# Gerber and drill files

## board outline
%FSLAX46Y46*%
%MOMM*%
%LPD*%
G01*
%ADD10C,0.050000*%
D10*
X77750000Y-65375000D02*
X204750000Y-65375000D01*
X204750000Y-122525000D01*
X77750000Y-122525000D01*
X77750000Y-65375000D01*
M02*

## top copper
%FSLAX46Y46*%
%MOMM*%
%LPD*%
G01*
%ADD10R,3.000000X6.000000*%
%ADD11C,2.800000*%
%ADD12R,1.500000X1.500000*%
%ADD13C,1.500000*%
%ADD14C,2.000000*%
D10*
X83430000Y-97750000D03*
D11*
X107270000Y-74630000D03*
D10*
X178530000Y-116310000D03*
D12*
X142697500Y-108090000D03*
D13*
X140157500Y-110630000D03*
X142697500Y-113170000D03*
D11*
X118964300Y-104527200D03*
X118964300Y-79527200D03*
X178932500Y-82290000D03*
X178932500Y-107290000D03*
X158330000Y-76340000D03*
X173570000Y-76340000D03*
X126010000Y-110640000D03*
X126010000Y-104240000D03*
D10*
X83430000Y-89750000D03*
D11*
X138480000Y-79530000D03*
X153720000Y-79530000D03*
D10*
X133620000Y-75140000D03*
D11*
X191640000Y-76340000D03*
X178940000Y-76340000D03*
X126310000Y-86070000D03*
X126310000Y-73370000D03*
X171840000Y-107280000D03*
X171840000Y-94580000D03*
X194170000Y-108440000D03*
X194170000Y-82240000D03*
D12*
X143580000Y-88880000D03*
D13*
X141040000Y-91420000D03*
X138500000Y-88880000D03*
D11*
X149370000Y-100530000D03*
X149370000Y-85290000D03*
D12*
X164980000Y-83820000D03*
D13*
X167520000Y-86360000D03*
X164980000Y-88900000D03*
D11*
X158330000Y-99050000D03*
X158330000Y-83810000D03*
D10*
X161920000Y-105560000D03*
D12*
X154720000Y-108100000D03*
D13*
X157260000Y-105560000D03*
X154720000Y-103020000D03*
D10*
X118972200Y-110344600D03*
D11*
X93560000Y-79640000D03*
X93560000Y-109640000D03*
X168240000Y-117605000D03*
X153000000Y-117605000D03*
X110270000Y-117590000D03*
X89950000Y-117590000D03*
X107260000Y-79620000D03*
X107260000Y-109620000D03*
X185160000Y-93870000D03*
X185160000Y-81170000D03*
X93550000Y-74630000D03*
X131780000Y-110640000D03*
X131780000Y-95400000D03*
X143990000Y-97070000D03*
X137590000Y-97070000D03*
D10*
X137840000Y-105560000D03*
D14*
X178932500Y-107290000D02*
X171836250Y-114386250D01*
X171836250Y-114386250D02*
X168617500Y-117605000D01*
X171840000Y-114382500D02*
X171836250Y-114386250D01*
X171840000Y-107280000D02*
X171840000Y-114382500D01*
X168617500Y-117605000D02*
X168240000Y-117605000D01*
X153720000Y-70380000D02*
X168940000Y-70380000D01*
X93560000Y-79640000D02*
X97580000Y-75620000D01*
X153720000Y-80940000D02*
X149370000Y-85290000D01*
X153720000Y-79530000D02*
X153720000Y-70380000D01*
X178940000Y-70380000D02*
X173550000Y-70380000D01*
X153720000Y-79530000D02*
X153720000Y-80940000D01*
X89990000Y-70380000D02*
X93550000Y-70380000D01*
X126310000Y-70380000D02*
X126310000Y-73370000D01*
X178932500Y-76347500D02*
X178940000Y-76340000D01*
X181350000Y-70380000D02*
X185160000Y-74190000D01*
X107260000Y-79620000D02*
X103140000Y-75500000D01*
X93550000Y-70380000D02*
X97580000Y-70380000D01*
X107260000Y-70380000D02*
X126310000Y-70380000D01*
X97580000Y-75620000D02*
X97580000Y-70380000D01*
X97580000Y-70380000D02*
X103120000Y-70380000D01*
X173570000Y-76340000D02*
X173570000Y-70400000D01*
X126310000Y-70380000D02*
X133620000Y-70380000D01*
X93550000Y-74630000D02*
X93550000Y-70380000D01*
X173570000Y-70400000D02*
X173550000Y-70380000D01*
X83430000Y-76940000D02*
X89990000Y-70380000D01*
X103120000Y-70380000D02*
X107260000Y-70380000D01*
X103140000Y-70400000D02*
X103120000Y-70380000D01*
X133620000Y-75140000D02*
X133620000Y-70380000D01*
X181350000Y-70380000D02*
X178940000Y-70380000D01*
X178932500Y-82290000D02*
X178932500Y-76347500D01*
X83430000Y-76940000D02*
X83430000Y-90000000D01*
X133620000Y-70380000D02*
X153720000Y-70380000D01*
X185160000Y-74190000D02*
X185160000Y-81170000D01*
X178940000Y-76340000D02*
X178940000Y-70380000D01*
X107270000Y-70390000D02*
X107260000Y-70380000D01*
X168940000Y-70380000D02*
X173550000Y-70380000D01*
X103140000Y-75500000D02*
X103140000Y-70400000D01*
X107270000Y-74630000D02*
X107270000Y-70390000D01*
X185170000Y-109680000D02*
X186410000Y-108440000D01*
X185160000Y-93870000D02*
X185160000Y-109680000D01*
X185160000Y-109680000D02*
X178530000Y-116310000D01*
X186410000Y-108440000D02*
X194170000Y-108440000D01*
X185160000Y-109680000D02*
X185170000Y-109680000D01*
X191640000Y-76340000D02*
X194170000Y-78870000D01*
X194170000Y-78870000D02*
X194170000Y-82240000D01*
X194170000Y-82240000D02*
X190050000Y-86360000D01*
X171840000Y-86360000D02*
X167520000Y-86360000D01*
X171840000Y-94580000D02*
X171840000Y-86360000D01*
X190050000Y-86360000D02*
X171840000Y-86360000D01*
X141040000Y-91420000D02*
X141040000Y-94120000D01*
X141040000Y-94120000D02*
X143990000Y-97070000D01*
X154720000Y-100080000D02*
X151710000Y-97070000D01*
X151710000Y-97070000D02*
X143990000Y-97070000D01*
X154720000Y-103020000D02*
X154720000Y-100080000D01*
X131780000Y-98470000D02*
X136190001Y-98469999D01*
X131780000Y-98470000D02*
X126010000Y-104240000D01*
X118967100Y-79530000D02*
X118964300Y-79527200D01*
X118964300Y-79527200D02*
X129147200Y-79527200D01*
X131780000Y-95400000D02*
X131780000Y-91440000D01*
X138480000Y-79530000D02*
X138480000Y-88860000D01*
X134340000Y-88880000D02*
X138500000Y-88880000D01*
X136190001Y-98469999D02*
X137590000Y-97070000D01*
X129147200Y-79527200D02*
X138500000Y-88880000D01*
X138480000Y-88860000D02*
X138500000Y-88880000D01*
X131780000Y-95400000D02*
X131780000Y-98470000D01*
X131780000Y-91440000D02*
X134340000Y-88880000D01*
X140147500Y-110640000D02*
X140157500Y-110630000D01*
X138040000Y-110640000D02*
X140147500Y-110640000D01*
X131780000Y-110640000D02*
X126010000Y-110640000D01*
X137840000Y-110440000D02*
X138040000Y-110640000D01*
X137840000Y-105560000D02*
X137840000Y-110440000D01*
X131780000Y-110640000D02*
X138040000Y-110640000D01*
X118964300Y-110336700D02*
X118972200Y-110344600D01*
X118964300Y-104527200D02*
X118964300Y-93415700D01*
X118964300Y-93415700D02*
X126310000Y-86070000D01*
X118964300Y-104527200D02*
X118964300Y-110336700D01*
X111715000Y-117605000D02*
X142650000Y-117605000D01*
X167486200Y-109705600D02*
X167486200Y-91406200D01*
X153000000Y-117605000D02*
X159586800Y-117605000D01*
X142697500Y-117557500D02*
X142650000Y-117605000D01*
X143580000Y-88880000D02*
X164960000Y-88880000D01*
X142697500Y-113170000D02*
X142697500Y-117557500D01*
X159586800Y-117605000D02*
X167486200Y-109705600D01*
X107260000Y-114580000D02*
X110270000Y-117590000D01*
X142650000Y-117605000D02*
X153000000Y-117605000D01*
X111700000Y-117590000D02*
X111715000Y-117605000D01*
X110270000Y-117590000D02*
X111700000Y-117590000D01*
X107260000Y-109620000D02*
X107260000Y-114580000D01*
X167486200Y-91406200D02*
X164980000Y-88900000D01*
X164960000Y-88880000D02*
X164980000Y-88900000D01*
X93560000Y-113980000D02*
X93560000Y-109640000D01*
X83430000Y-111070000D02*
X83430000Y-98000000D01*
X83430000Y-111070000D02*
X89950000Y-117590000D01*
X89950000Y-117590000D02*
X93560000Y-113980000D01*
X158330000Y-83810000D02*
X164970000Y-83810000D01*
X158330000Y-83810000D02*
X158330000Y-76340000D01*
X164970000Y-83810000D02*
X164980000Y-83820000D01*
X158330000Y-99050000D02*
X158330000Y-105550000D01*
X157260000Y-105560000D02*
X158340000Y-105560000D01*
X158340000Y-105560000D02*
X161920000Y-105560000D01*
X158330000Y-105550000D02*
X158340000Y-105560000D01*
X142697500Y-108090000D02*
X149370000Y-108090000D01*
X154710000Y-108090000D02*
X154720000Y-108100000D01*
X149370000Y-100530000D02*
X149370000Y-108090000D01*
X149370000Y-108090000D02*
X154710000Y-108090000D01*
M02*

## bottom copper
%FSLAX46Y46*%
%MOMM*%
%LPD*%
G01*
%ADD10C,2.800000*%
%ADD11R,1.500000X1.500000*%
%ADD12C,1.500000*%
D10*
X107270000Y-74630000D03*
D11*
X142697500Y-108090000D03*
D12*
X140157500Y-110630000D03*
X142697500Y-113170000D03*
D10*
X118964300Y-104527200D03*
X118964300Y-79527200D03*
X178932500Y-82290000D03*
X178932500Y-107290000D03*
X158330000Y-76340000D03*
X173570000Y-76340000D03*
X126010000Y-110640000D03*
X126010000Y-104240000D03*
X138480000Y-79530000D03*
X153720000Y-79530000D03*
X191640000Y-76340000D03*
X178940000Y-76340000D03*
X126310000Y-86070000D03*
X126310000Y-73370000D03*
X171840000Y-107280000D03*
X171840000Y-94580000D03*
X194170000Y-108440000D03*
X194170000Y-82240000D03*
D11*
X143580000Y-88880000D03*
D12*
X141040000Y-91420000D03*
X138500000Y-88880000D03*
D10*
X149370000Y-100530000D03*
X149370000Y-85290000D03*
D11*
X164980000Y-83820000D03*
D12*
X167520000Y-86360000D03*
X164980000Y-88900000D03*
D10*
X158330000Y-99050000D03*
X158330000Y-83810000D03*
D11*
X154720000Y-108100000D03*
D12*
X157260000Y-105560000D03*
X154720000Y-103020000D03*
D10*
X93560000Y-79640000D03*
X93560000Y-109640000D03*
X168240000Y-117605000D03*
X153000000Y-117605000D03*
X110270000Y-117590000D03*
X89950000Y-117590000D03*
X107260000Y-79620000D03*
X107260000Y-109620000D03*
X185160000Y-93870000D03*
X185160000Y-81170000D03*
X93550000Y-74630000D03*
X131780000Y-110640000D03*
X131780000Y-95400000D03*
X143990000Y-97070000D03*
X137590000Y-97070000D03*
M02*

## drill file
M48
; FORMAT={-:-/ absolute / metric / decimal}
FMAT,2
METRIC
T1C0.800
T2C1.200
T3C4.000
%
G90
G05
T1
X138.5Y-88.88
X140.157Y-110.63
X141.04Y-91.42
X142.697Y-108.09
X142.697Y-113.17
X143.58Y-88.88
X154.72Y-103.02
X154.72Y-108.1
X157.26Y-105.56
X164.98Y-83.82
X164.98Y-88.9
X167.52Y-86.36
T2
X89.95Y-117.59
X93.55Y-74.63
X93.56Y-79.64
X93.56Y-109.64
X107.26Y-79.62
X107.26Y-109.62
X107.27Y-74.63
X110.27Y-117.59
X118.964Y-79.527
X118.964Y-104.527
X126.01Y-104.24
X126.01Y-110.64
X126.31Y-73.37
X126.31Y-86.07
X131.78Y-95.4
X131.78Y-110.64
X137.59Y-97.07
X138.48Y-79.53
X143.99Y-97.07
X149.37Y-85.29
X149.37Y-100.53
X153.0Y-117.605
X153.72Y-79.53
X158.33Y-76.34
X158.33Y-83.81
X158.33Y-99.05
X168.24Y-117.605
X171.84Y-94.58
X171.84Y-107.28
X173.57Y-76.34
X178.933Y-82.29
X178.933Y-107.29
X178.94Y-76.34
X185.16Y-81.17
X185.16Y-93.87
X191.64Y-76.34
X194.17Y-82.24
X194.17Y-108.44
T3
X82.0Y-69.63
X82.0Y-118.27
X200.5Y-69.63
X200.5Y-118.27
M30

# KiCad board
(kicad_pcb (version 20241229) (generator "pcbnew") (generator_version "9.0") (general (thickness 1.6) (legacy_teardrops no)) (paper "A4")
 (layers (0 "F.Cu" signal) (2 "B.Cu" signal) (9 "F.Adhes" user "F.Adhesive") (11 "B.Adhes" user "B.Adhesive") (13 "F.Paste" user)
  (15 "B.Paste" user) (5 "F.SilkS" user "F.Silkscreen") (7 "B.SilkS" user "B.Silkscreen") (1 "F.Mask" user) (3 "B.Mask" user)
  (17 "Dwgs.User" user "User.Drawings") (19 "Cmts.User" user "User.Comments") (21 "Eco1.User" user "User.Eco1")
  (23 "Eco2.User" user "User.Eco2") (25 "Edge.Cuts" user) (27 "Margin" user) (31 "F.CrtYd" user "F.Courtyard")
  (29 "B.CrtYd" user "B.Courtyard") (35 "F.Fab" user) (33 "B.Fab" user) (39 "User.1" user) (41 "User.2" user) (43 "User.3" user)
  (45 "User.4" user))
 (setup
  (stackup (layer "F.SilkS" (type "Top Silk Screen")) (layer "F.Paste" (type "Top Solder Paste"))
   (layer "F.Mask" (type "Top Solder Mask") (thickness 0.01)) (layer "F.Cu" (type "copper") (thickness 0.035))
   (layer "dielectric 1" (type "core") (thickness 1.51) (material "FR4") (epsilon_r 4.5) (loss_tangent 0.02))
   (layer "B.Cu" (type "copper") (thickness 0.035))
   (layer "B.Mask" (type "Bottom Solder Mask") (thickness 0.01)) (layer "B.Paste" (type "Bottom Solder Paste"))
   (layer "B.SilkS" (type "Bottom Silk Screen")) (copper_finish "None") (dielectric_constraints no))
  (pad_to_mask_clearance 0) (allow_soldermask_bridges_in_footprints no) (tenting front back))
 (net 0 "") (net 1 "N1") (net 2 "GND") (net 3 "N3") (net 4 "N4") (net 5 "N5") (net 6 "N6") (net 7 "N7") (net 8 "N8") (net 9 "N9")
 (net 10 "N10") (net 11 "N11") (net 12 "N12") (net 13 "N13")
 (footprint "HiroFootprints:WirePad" (layer "F.Cu") (at 83.43 98)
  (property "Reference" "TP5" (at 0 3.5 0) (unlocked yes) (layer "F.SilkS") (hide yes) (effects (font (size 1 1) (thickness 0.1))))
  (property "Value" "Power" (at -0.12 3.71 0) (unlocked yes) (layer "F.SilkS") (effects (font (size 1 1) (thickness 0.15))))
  (pad "1" smd rect (at 0 -0.25) (size 3 6) (layers "F.Cu" "F.Mask" "F.Paste") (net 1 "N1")))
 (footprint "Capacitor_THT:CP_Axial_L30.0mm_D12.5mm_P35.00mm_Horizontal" (layer "F.Cu") (at 107.27 74.63 -90)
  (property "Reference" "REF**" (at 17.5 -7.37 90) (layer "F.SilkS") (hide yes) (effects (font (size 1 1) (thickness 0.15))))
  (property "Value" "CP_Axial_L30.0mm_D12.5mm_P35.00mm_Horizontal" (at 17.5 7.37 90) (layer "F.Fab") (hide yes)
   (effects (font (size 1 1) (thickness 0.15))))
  (pad "1" thru_hole circle (at 0 0 270) (size 2.8 2.8) (drill 1.2) (layers "*.Cu" "*.Mask") (remove_unused_layers no) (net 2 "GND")))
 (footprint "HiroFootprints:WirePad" (layer "F.Cu") (at 178.53 116.56)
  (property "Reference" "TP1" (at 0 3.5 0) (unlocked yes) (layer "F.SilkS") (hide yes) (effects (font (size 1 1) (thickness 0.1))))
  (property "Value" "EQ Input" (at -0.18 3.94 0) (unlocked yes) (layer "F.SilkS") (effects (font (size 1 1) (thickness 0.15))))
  (pad "1" smd rect (at 0 -0.25) (size 3 6) (layers "F.Cu" "F.Mask" "F.Paste") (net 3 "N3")))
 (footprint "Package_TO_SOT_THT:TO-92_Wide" (layer "F.Cu") (at 142.6975 108.09 -90)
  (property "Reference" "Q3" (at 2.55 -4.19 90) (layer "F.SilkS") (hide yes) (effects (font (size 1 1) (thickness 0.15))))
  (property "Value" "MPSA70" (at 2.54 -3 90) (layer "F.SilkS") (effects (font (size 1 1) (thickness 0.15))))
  (pad "1" thru_hole rect (at 0 0 270) (size 1.5 1.5) (drill 0.8) (layers "*.Cu" "*.Mask") (remove_unused_layers no) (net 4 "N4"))
  (pad "2" thru_hole circle (at 2.54 2.54 270) (size 1.5 1.5) (drill 0.8) (layers "*.Cu" "*.Mask") (remove_unused_layers no) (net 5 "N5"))
  (pad "3" thru_hole circle (at 5.08 0 270) (size 1.5 1.5) (drill 0.8) (layers "*.Cu" "*.Mask") (remove_unused_layers no) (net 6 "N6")))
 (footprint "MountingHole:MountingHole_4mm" (layer "F.Cu") (at 200.5 118.27)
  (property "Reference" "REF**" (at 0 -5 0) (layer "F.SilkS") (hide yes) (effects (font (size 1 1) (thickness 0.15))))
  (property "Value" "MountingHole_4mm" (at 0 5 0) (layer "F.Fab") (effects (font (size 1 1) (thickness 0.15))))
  (pad "" np_thru_hole circle (at 0 0) (size 4 4) (drill 4) (layers "*.Cu" "*.Mask")))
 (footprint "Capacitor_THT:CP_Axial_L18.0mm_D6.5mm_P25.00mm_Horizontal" (layer "F.Cu") (at 118.9643 104.5272 90)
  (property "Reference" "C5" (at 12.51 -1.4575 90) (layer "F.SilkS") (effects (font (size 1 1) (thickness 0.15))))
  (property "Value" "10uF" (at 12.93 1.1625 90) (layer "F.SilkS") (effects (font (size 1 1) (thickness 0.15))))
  (pad "1" thru_hole circle (at 0 0 90) (size 2.8 2.8) (drill 1.2) (layers "*.Cu" "*.Mask") (remove_unused_layers no) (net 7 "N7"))
  (pad "2" thru_hole circle (at 25 0 90) (size 2.8 2.8) (drill 1.2) (layers "*.Cu" "*.Mask") (remove_unused_layers no) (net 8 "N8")))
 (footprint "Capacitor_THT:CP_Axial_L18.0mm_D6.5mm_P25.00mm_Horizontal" (layer "F.Cu") (at 178.9325 82.29 -90)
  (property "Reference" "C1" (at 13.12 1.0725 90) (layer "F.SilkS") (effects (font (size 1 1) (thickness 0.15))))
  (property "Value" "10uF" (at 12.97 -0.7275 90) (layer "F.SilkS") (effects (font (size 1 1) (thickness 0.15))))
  (pad "1" thru_hole circle (at 0 0 270) (size 2.8 2.8) (drill 1.2) (layers "*.Cu" "*.Mask") (remove_unused_layers no) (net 2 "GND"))
  (pad "2" thru_hole circle (at 25 0 270) (size 2.8 2.8) (drill 1.2) (layers "*.Cu" "*.Mask") (remove_unused_layers no) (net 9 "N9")))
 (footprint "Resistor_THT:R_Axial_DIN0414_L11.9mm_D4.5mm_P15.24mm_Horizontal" (layer "F.Cu") (at 158.33 76.34)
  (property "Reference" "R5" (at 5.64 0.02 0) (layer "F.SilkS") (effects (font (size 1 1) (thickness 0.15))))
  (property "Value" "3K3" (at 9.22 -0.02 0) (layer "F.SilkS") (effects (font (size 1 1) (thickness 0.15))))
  (pad "1" thru_hole circle (at 0 0) (size 2.8 2.8) (drill 1.2) (layers "*.Cu" "*.Mask") (remove_unused_layers no) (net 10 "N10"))
  (pad "2" thru_hole circle (at 15.24 0) (size 2.8 2.8) (drill 1.2) (layers "*.Cu" "*.Mask") (remove_unused_layers no) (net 2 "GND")))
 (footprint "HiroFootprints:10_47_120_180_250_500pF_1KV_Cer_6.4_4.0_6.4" (layer "F.Cu") (at 126.01 110.64 90)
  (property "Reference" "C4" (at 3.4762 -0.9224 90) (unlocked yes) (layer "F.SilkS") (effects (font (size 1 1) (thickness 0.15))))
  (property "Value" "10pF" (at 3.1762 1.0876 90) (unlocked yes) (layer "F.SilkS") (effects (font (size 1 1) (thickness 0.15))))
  (pad "1" thru_hole circle (at 0 0 90) (size 2.8 2.8) (drill 1.2) (layers "*.Cu" "*.Mask") (remove_unused_layers no) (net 5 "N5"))
  (pad "2" thru_hole circle (at 6.4 0 90) (size 2.8 2.8) (drill 1.2) (layers "*.Cu" "*.Mask") (remove_unused_layers no) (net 8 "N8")))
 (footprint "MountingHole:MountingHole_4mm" (layer "F.Cu") (at 200.5 69.63)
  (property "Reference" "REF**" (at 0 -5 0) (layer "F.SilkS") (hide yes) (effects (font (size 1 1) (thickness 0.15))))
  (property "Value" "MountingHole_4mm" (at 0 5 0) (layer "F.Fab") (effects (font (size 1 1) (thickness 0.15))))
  (pad "" np_thru_hole circle (at 0 0) (size 4 4) (drill 4) (layers "*.Cu" "*.Mask")))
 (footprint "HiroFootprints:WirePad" (layer "F.Cu") (at 83.43 90)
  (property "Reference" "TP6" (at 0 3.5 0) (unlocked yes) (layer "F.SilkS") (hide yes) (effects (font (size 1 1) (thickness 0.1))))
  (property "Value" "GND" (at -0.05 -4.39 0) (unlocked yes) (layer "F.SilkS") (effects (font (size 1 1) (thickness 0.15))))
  (pad "1" smd rect (at 0 -0.25) (size 3 6) (layers "F.Cu" "F.Mask" "F.Paste") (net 2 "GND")))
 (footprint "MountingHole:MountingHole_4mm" (layer "F.Cu") (at 82 69.63)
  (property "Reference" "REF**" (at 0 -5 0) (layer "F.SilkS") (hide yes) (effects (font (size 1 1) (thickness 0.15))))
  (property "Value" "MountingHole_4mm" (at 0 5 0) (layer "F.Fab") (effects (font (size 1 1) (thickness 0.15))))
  (pad "" np_thru_hole circle (at 0 0) (size 4 4) (drill 4) (layers "*.Cu" "*.Mask")))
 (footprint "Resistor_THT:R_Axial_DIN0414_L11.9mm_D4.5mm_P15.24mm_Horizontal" (layer "F.Cu") (at 138.48 79.53)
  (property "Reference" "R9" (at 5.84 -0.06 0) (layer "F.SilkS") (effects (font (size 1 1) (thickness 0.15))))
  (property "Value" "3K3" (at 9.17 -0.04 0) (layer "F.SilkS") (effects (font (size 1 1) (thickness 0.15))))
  (pad "1" thru_hole circle (at 0 0) (size 2.8 2.8) (drill 1.2) (layers "*.Cu" "*.Mask") (remove_unused_layers no) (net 8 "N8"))
  (pad "2" thru_hole circle (at 15.24 0) (size 2.8 2.8) (drill 1.2) (layers "*.Cu" "*.Mask") (remove_unused_layers no) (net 2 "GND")))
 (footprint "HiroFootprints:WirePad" (layer "F.Cu") (at 133.62 75.39)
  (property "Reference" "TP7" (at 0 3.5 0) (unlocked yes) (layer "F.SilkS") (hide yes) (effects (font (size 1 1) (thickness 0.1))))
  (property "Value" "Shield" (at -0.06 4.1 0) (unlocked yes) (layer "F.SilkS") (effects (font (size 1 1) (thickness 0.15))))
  (pad "1" smd rect (at 0 -0.25) (size 3 6) (layers "F.Cu" "F.Mask" "F.Paste") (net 2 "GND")))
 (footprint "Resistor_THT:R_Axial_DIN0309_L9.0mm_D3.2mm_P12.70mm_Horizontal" (layer "F.Cu") (at 191.64 76.34 180)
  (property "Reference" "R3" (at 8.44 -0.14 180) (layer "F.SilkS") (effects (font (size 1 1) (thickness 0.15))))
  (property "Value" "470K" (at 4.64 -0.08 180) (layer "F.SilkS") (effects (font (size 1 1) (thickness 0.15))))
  (pad "1" thru_hole circle (at 0 0 180) (size 2.8 2.8) (drill 1.2) (layers "*.Cu" "*.Mask") (remove_unused_layers no) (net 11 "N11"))
  (pad "2" thru_hole circle (at 12.7 0 180) (size 2.8 2.8) (drill 1.2) (layers "*.Cu" "*.Mask") (remove_unused_layers no) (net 2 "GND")))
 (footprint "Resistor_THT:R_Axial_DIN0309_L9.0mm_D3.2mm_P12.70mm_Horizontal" (layer "F.Cu") (at 126.31 86.07 90)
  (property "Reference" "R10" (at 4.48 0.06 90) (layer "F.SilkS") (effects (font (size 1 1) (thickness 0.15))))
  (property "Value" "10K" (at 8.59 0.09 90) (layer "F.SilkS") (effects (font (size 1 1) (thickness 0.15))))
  (pad "1" thru_hole circle (at 0 0 90) (size 2.8 2.8) (drill 1.2) (layers "*.Cu" "*.Mask") (remove_unused_layers no) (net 7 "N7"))
  (pad "2" thru_hole circle (at 12.7 0 90) (size 2.8 2.8) (drill 1.2) (layers "*.Cu" "*.Mask") (remove_unused_layers no) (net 2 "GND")))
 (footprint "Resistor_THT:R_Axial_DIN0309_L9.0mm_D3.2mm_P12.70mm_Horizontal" (layer "F.Cu") (at 171.84 107.28 90)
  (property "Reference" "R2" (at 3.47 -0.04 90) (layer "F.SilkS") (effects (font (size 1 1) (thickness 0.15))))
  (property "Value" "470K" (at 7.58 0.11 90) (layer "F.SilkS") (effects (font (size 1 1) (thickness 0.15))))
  (pad "1" thru_hole circle (at 0 0 90) (size 2.8 2.8) (drill 1.2) (layers "*.Cu" "*.Mask") (remove_unused_layers no) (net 9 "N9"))
  (pad "2" thru_hole circle (at 12.7 0 90) (size 2.8 2.8) (drill 1.2) (layers "*.Cu" "*.Mask") (remove_unused_layers no) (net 11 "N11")))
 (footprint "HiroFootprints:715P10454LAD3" (layer "F.Cu") (at 194.17 108.44 90)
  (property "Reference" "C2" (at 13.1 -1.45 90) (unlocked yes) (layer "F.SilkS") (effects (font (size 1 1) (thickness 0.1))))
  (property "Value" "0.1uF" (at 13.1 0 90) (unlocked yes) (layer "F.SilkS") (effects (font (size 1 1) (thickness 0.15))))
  (pad "1" thru_hole circle (at 0 0 90) (size 2.8 2.8) (drill 1.2) (layers "*.Cu" "*.Mask") (remove_unused_layers no) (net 3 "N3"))
  (pad "2" thru_hole circle (at 26.2 0 90) (size 2.8 2.8) (drill 1.2) (layers "*.Cu" "*.Mask") (remove_unused_layers no) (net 11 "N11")))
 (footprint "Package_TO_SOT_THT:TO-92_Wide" (layer "F.Cu") (at 143.58 88.88 180)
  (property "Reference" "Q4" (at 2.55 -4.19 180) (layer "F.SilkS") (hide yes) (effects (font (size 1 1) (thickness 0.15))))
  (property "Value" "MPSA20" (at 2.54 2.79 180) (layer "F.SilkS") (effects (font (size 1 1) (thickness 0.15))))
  (pad "1" thru_hole rect (at 0 0 180) (size 1.5 1.5) (drill 0.8) (layers "*.Cu" "*.Mask") (remove_unused_layers no) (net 6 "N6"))
  (pad "2" thru_hole circle (at 2.54 -2.54 180) (size 1.5 1.5) (drill 0.8) (layers "*.Cu" "*.Mask") (remove_unused_layers no) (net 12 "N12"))
  (pad "3" thru_hole circle (at 5.08 0 180) (size 1.5 1.5) (drill 0.8) (layers "*.Cu" "*.Mask") (remove_unused_layers no) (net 8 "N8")))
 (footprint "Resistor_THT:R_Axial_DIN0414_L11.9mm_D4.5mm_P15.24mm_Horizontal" (layer "F.Cu") (at 149.37 100.53 90)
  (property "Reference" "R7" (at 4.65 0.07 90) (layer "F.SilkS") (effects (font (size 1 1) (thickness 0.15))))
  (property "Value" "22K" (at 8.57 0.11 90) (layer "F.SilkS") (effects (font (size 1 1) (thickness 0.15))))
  (pad "1" thru_hole circle (at 0 0 90) (size 2.8 2.8) (drill 1.2) (layers "*.Cu" "*.Mask") (remove_unused_layers no) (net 4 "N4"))
  (pad "2" thru_hole circle (at 15.24 0 90) (size 2.8 2.8) (drill 1.2) (layers "*.Cu" "*.Mask") (remove_unused_layers no) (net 2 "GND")))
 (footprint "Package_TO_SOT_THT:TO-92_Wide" (layer "F.Cu") (at 164.98 83.82 -90)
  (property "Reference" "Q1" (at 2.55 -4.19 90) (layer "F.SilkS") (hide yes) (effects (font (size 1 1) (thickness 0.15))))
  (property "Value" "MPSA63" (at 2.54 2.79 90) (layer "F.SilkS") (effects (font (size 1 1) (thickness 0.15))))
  (pad "1" thru_hole rect (at 0 0 270) (size 1.5 1.5) (drill 0.8) (layers "*.Cu" "*.Mask") (remove_unused_layers no) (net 10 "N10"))
  (pad "2" thru_hole circle (at 2.54 -2.54 270) (size 1.5 1.5) (drill 0.8) (layers "*.Cu" "*.Mask") (remove_unused_layers no) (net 11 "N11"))
  (pad "3" thru_hole circle (at 5.08 0 270) (size 1.5 1.5) (drill 0.8) (layers "*.Cu" "*.Mask") (remove_unused_layers no) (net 6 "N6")))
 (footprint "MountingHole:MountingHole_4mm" (layer "F.Cu") (at 82 118.27)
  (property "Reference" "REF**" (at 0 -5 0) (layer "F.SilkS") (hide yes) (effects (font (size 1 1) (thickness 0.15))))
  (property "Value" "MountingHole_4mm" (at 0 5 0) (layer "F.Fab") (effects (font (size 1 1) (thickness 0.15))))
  (pad "" np_thru_hole circle (at 0 0) (size 4 4) (drill 4) (layers "*.Cu" "*.Mask")))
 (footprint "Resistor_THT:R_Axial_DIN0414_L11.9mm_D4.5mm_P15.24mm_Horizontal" (layer "F.Cu") (at 158.33 99.05 90)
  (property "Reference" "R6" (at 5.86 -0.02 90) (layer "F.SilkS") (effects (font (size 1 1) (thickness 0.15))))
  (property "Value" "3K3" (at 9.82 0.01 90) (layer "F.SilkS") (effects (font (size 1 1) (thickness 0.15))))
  (pad "1" thru_hole circle (at 0 0 90) (size 2.8 2.8) (drill 1.2) (layers "*.Cu" "*.Mask") (remove_unused_layers no) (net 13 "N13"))
  (pad "2" thru_hole circle (at 15.24 0 90) (size 2.8 2.8) (drill 1.2) (layers "*.Cu" "*.Mask") (remove_unused_layers no) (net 10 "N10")))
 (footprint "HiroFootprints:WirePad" (layer "F.Cu") (at 161.92 105.81)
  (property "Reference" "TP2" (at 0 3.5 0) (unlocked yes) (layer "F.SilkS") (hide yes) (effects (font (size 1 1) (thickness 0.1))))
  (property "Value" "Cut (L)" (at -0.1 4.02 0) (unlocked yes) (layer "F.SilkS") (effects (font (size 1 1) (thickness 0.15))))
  (pad "1" smd rect (at 0 -0.25) (size 3 6) (layers "F.Cu" "F.Mask" "F.Paste") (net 13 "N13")))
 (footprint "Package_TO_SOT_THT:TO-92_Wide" (layer "F.Cu") (at 154.72 108.1 90)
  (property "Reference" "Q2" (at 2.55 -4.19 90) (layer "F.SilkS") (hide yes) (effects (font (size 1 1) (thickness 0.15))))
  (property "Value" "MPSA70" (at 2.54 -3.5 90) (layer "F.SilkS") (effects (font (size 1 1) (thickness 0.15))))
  (pad "1" thru_hole rect (at 0 0 90) (size 1.5 1.5) (drill 0.8) (layers "*.Cu" "*.Mask") (remove_unused_layers no) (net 4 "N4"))
  (pad "2" thru_hole circle (at 2.54 2.54 90) (size 1.5 1.5) (drill 0.8) (layers "*.Cu" "*.Mask") (remove_unused_layers no) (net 13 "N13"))
  (pad "3" thru_hole circle (at 5.08 0 90) (size 1.5 1.5) (drill 0.8) (layers "*.Cu" "*.Mask") (remove_unused_layers no) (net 12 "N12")))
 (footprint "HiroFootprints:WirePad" (layer "F.Cu") (at 118.9722 110.5946)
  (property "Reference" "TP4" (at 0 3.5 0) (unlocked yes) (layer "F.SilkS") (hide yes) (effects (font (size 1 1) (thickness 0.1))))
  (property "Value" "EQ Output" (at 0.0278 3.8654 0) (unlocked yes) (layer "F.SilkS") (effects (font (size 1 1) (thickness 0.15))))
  (pad "1" smd rect (at 0 -0.25) (size 3 6) (layers "F.Cu" "F.Mask" "F.Paste") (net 7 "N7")))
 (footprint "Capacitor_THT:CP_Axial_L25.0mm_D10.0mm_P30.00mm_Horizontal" (layer "F.Cu") (at 93.56 79.64 -90)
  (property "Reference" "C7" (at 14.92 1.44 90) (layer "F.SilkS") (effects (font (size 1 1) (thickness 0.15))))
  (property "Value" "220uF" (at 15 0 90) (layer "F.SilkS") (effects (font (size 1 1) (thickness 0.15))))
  (pad "1" thru_hole circle (at 0 0 270) (size 2.8 2.8) (drill 1.2) (layers "*.Cu" "*.Mask") (remove_unused_layers no) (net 2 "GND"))
  (pad "2" thru_hole circle (at 30 0 270) (size 2.8 2.8) (drill 1.2) (layers "*.Cu" "*.Mask") (remove_unused_layers no) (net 1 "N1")))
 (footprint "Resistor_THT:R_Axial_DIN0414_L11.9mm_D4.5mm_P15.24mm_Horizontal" (layer "F.Cu") (at 168.24 117.605 180)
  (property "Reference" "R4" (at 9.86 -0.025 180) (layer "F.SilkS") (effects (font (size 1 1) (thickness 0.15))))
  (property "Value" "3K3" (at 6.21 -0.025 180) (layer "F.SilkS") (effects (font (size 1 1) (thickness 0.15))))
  (pad "1" thru_hole circle (at 0 0 180) (size 2.8 2.8) (drill 1.2) (layers "*.Cu" "*.Mask") (remove_unused_layers no) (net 9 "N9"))
  (pad "2" thru_hole circle (at 15.24 0 180) (size 2.8 2.8) (drill 1.2) (layers "*.Cu" "*.Mask") (remove_unused_layers no) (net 6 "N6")))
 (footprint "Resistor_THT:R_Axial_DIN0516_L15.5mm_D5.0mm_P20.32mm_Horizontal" (layer "F.Cu") (at 110.27 117.59 180)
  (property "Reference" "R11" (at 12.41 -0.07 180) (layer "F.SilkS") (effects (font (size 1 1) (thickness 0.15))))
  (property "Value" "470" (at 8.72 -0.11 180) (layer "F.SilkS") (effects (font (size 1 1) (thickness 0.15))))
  (pad "1" thru_hole circle (at 0 0 180) (size 2.8 2.8) (drill 1.2) (layers "*.Cu" "*.Mask") (remove_unused_layers no) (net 6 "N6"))
  (pad "2" thru_hole circle (at 20.32 0 180) (size 2.8 2.8) (drill 1.2) (layers "*.Cu" "*.Mask") (remove_unused_layers no) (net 1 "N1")))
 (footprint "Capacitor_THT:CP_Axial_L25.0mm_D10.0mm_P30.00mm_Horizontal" (layer "F.Cu") (at 107.26 79.62 -90)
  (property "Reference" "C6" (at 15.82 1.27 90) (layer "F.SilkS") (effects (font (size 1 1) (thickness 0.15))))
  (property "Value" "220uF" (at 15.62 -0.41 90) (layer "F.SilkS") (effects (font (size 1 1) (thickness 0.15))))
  (pad "1" thru_hole circle (at 0 0 270) (size 2.8 2.8) (drill 1.2) (layers "*.Cu" "*.Mask") (remove_unused_layers no) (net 2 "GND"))
  (pad "2" thru_hole circle (at 30 0 270) (size 2.8 2.8) (drill 1.2) (layers "*.Cu" "*.Mask") (remove_unused_layers no) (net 6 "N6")))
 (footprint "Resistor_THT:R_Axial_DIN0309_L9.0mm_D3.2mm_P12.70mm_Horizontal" (layer "F.Cu") (at 185.16 93.87 90)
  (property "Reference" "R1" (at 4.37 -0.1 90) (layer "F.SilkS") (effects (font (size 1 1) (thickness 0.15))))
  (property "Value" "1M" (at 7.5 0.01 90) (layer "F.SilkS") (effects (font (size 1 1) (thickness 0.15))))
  (pad "1" thru_hole circle (at 0 0 90) (size 2.8 2.8) (drill 1.2) (layers "*.Cu" "*.Mask") (remove_unused_layers no) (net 3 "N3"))
  (pad "2" thru_hole circle (at 12.7 0 90) (size 2.8 2.8) (drill 1.2) (layers "*.Cu" "*.Mask") (remove_unused_layers no) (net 2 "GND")))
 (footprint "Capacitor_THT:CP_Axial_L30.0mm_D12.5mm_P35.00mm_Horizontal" (layer "F.Cu") (at 93.55 74.63 -90)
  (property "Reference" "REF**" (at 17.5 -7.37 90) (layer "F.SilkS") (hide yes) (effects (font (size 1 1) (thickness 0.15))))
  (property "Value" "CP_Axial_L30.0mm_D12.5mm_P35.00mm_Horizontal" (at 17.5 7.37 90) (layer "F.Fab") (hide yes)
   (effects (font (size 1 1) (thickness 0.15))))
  (pad "1" thru_hole circle (at 0 0 270) (size 2.8 2.8) (drill 1.2) (layers "*.Cu" "*.Mask") (remove_unused_layers no) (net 2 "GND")))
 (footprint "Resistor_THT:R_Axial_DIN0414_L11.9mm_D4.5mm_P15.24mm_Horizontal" (layer "F.Cu") (at 131.78 110.64 90)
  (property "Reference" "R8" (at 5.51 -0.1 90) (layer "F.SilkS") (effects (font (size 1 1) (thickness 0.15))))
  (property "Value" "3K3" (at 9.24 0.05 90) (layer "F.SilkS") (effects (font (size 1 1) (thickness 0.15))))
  (pad "1" thru_hole circle (at 0 0 90) (size 2.8 2.8) (drill 1.2) (layers "*.Cu" "*.Mask") (remove_unused_layers no) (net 5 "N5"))
  (pad "2" thru_hole circle (at 15.24 0 90) (size 2.8 2.8) (drill 1.2) (layers "*.Cu" "*.Mask") (remove_unused_layers no) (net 8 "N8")))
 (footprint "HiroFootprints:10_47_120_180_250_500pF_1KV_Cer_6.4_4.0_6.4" (layer "F.Cu") (at 143.99 97.07 180)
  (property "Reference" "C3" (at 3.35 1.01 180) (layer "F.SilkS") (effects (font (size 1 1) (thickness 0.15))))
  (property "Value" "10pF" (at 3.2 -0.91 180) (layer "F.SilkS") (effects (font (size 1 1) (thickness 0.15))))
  (pad "1" thru_hole circle (at 0 0 180) (size 2.8 2.8) (drill 1.2) (layers "*.Cu" "*.Mask") (remove_unused_layers no) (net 12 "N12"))
  (pad "2" thru_hole circle (at 6.4 0 180) (size 2.8 2.8) (drill 1.2) (layers "*.Cu" "*.Mask") (remove_unused_layers no) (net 8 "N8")))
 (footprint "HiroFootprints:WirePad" (layer "F.Cu") (at 137.84 105.81)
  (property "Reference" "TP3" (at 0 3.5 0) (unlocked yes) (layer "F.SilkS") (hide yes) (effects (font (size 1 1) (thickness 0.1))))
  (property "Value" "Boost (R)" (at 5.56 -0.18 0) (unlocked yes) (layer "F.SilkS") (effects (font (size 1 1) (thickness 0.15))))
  (pad "1" smd rect (at 0 -0.25) (size 3 6) (layers "F.Cu" "F.Mask" "F.Paste") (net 5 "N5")))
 (gr_rect (start 77.75 65.375) (end 204.75 122.525) (stroke (width 0.05) (type solid)) (fill no) (layer "Edge.Cuts"))
 (segment (start 178.9325 107.29) (end 171.83625 114.38625) (width 2) (layer "F.Cu") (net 9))
 (segment (start 171.83625 114.38625) (end 168.6175 117.605) (width 2) (layer "F.Cu") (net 9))
 (segment (start 171.84 114.3825) (end 171.83625 114.38625) (width 2) (layer "F.Cu") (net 9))
 (segment (start 171.84 107.28) (end 171.84 114.3825) (width 2) (layer "F.Cu") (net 9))
 (segment (start 168.6175 117.605) (end 168.24 117.605) (width 2) (layer "F.Cu") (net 9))
 (segment (start 153.72 70.38) (end 168.94 70.38) (width 2) (layer "F.Cu") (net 2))
 (segment (start 93.56 79.64) (end 97.58 75.62) (width 2) (layer "F.Cu") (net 2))
 (segment (start 153.72 80.94) (end 149.37 85.29) (width 2) (layer "F.Cu") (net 2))
 (segment (start 153.72 79.53) (end 153.72 70.38) (width 2) (layer "F.Cu") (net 2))
 (segment (start 178.94 70.38) (end 173.55 70.38) (width 2) (layer "F.Cu") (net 2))
 (segment (start 153.72 79.53) (end 153.72 80.94) (width 2) (layer "F.Cu") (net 2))
 (segment (start 89.99 70.38) (end 93.55 70.38) (width 2) (layer "F.Cu") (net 2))
 (segment (start 126.31 70.38) (end 126.31 73.37) (width 2) (layer "F.Cu") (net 2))
 (segment (start 178.9325 76.3475) (end 178.94 76.34) (width 2) (layer "F.Cu") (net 2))
 (segment (start 181.35 70.38) (end 185.16 74.19) (width 2) (layer "F.Cu") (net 2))
 (segment (start 107.26 79.62) (end 103.14 75.5) (width 2) (layer "F.Cu") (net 2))
 (segment (start 93.55 70.38) (end 97.58 70.38) (width 2) (layer "F.Cu") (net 2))
 (segment (start 107.26 70.38) (end 126.31 70.38) (width 2) (layer "F.Cu") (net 2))
 (segment (start 97.58 75.62) (end 97.58 70.38) (width 2) (layer "F.Cu") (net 2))
 (segment (start 97.58 70.38) (end 103.12 70.38) (width 2) (layer "F.Cu") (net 2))
 (segment (start 173.57 76.34) (end 173.57 70.4) (width 2) (layer "F.Cu") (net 2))
 (segment (start 126.31 70.38) (end 133.62 70.38) (width 2) (layer "F.Cu") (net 2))
 (segment (start 93.55 74.63) (end 93.55 70.38) (width 2) (layer "F.Cu") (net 2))
 (segment (start 173.57 70.4) (end 173.55 70.38) (width 2) (layer "F.Cu") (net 2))
 (segment (start 83.43 76.94) (end 89.99 70.38) (width 2) (layer "F.Cu") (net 2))
 (segment (start 103.12 70.38) (end 107.26 70.38) (width 2) (layer "F.Cu") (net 2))
 (segment (start 103.14 70.4) (end 103.12 70.38) (width 2) (layer "F.Cu") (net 2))
 (segment (start 133.62 75.14) (end 133.62 70.38) (width 2) (layer "F.Cu") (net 2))
 (segment (start 181.35 70.38) (end 178.94 70.38) (width 2) (layer "F.Cu") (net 2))
 (segment (start 178.9325 82.29) (end 178.9325 76.3475) (width 2) (layer "F.Cu") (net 2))
 (segment (start 83.43 76.94) (end 83.43 90) (width 2) (layer "F.Cu") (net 2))
 (segment (start 133.62 70.38) (end 153.72 70.38) (width 2) (layer "F.Cu") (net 2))
 (segment (start 185.16 74.19) (end 185.16 81.17) (width 2) (layer "F.Cu") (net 2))
 (segment (start 178.94 76.34) (end 178.94 70.38) (width 2) (layer "F.Cu") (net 2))
 (segment (start 107.27 70.39) (end 107.26 70.38) (width 2) (layer "F.Cu") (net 2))
 (segment (start 168.94 70.38) (end 173.55 70.38) (width 2) (layer "F.Cu") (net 2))
 (segment (start 103.14 75.5) (end 103.14 70.4) (width 2) (layer "F.Cu") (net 2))
 (segment (start 107.27 74.63) (end 107.27 70.39) (width 2) (layer "F.Cu") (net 2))
 (segment (start 185.17 109.68) (end 186.41 108.44) (width 2) (layer "F.Cu") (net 3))
 (segment (start 185.16 93.87) (end 185.16 109.68) (width 2) (layer "F.Cu") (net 3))
 (segment (start 185.16 109.68) (end 178.53 116.31) (width 2) (layer "F.Cu") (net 3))
 (segment (start 186.41 108.44) (end 194.17 108.44) (width 2) (layer "F.Cu") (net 3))
 (segment (start 185.16 109.68) (end 185.17 109.68) (width 2) (layer "F.Cu") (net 3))
 (segment (start 191.64 76.34) (end 194.17 78.87) (width 2) (layer "F.Cu") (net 11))
 (segment (start 194.17 78.87) (end 194.17 82.24) (width 2) (layer "F.Cu") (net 11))
 (segment (start 194.17 82.24) (end 190.05 86.36) (width 2) (layer "F.Cu") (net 11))
 (segment (start 171.84 86.36) (end 167.52 86.36) (width 2) (layer "F.Cu") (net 11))
 (segment (start 171.84 94.58) (end 171.84 86.36) (width 2) (layer "F.Cu") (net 11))
 (segment (start 190.05 86.36) (end 171.84 86.36) (width 2) (layer "F.Cu") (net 11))
 (segment (start 141.04 91.42) (end 141.04 94.12) (width 2) (layer "F.Cu") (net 12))
 (segment (start 141.04 94.12) (end 143.99 97.07) (width 2) (layer "F.Cu") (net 12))
 (segment (start 154.72 100.08) (end 151.71 97.07) (width 2) (layer "F.Cu") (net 12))
 (segment (start 151.71 97.07) (end 143.99 97.07) (width 2) (layer "F.Cu") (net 12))
 (segment (start 154.72 103.02) (end 154.72 100.08) (width 2) (layer "F.Cu") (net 12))
 (segment (start 131.78 98.47) (end 136.190001 98.469999) (width 2) (layer "F.Cu") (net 8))
 (segment (start 131.78 98.47) (end 126.01 104.24) (width 2) (layer "F.Cu") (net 8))
 (segment (start 118.9671 79.53) (end 118.9643 79.5272) (width 2) (layer "F.Cu") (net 8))
 (segment (start 118.9643 79.5272) (end 129.1472 79.5272) (width 2) (layer "F.Cu") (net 8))
 (segment (start 131.78 95.4) (end 131.78 91.44) (width 2) (layer "F.Cu") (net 8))
 (segment (start 138.48 79.53) (end 138.48 88.86) (width 2) (layer "F.Cu") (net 8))
 (segment (start 134.34 88.88) (end 138.5 88.88) (width 2) (layer "F.Cu") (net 8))
 (segment (start 136.190001 98.469999) (end 137.59 97.07) (width 2) (layer "F.Cu") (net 8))
 (segment (start 129.1472 79.5272) (end 138.5 88.88) (width 2) (layer "F.Cu") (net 8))
 (segment (start 138.48 88.86) (end 138.5 88.88) (width 2) (layer "F.Cu") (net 8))
 (segment (start 131.78 95.4) (end 131.78 98.47) (width 2) (layer "F.Cu") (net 8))
 (segment (start 131.78 91.44) (end 134.34 88.88) (width 2) (layer "F.Cu") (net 8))
 (segment (start 140.1475 110.64) (end 140.1575 110.63) (width 2) (layer "F.Cu") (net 5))
 (segment (start 138.04 110.64) (end 140.1475 110.64) (width 2) (layer "F.Cu") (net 5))
 (segment (start 131.78 110.64) (end 126.01 110.64) (width 2) (layer "F.Cu") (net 5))
 (segment (start 137.84 110.44) (end 138.04 110.64) (width 2) (layer "F.Cu") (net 5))
 (segment (start 137.84 105.56) (end 137.84 110.44) (width 2) (layer "F.Cu") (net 5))
 (segment (start 131.78 110.64) (end 138.04 110.64) (width 2) (layer "F.Cu") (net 5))
 (segment (start 118.9643 110.3367) (end 118.9722 110.3446) (width 2) (layer "F.Cu") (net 7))
 (segment (start 118.9643 104.5272) (end 118.9643 93.4157) (width 2) (layer "F.Cu") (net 7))
 (segment (start 118.9643 93.4157) (end 126.31 86.07) (width 2) (layer "F.Cu") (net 7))
 (segment (start 118.9643 104.5272) (end 118.9643 110.3367) (width 2) (layer "F.Cu") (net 7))
 (segment (start 111.715 117.605) (end 142.65 117.605) (width 2) (layer "F.Cu") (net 6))
 (segment (start 167.4862 109.7056) (end 167.4862 91.4062) (width 2) (layer "F.Cu") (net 6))
 (segment (start 153 117.605) (end 159.5868 117.605) (width 2) (layer "F.Cu") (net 6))
 (segment (start 142.6975 117.5575) (end 142.65 117.605) (width 2) (layer "F.Cu") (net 6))
 (segment (start 143.58 88.88) (end 164.96 88.88) (width 2) (layer "F.Cu") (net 6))
 (segment (start 142.6975 113.17) (end 142.6975 117.5575) (width 2) (layer "F.Cu") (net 6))
 (segment (start 159.5868 117.605) (end 167.4862 109.7056) (width 2) (layer "F.Cu") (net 6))
 (segment (start 107.26 114.58) (end 110.27 117.59) (width 2) (layer "F.Cu") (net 6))
 (segment (start 142.65 117.605) (end 153 117.605) (width 2) (layer "F.Cu") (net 6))
 (segment (start 111.7 117.59) (end 111.715 117.605) (width 2) (layer "F.Cu") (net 6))
 (segment (start 110.27 117.59) (end 111.7 117.59) (width 2) (layer "F.Cu") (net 6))
 (segment (start 107.26 109.62) (end 107.26 114.58) (width 2) (layer "F.Cu") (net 6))
 (segment (start 167.4862 91.4062) (end 164.98 88.9) (width 2) (layer "F.Cu") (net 6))
 (segment (start 164.96 88.88) (end 164.98 88.9) (width 2) (layer "F.Cu") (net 6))
 (segment (start 93.56 113.98) (end 93.56 109.64) (width 2) (layer "F.Cu") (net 1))
 (segment (start 83.43 111.07) (end 83.43 98) (width 2) (layer "F.Cu") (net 1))
 (segment (start 83.43 111.07) (end 89.95 117.59) (width 2) (layer "F.Cu") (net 1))
 (segment (start 89.95 117.59) (end 93.56 113.98) (width 2) (layer "F.Cu") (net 1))
 (segment (start 158.33 83.81) (end 164.97 83.81) (width 2) (layer "F.Cu") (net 10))
 (segment (start 158.33 83.81) (end 158.33 76.34) (width 2) (layer "F.Cu") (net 10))
 (segment (start 164.97 83.81) (end 164.98 83.82) (width 2) (layer "F.Cu") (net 10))
 (segment (start 158.33 99.05) (end 158.33 105.55) (width 2) (layer "F.Cu") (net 13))
 (segment (start 157.26 105.56) (end 158.34 105.56) (width 2) (layer "F.Cu") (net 13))
 (segment (start 158.34 105.56) (end 161.92 105.56) (width 2) (layer "F.Cu") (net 13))
 (segment (start 158.33 105.55) (end 158.34 105.56) (width 2) (layer "F.Cu") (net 13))
 (segment (start 142.6975 108.09) (end 149.37 108.09) (width 2) (layer "F.Cu") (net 4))
 (segment (start 154.71 108.09) (end 154.72 108.1) (width 2) (layer "F.Cu") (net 4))
 (segment (start 149.37 100.53) (end 149.37 108.09) (width 2) (layer "F.Cu") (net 4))
 (segment (start 149.37 108.09) (end 154.71 108.09) (width 2) (layer "F.Cu") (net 4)))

